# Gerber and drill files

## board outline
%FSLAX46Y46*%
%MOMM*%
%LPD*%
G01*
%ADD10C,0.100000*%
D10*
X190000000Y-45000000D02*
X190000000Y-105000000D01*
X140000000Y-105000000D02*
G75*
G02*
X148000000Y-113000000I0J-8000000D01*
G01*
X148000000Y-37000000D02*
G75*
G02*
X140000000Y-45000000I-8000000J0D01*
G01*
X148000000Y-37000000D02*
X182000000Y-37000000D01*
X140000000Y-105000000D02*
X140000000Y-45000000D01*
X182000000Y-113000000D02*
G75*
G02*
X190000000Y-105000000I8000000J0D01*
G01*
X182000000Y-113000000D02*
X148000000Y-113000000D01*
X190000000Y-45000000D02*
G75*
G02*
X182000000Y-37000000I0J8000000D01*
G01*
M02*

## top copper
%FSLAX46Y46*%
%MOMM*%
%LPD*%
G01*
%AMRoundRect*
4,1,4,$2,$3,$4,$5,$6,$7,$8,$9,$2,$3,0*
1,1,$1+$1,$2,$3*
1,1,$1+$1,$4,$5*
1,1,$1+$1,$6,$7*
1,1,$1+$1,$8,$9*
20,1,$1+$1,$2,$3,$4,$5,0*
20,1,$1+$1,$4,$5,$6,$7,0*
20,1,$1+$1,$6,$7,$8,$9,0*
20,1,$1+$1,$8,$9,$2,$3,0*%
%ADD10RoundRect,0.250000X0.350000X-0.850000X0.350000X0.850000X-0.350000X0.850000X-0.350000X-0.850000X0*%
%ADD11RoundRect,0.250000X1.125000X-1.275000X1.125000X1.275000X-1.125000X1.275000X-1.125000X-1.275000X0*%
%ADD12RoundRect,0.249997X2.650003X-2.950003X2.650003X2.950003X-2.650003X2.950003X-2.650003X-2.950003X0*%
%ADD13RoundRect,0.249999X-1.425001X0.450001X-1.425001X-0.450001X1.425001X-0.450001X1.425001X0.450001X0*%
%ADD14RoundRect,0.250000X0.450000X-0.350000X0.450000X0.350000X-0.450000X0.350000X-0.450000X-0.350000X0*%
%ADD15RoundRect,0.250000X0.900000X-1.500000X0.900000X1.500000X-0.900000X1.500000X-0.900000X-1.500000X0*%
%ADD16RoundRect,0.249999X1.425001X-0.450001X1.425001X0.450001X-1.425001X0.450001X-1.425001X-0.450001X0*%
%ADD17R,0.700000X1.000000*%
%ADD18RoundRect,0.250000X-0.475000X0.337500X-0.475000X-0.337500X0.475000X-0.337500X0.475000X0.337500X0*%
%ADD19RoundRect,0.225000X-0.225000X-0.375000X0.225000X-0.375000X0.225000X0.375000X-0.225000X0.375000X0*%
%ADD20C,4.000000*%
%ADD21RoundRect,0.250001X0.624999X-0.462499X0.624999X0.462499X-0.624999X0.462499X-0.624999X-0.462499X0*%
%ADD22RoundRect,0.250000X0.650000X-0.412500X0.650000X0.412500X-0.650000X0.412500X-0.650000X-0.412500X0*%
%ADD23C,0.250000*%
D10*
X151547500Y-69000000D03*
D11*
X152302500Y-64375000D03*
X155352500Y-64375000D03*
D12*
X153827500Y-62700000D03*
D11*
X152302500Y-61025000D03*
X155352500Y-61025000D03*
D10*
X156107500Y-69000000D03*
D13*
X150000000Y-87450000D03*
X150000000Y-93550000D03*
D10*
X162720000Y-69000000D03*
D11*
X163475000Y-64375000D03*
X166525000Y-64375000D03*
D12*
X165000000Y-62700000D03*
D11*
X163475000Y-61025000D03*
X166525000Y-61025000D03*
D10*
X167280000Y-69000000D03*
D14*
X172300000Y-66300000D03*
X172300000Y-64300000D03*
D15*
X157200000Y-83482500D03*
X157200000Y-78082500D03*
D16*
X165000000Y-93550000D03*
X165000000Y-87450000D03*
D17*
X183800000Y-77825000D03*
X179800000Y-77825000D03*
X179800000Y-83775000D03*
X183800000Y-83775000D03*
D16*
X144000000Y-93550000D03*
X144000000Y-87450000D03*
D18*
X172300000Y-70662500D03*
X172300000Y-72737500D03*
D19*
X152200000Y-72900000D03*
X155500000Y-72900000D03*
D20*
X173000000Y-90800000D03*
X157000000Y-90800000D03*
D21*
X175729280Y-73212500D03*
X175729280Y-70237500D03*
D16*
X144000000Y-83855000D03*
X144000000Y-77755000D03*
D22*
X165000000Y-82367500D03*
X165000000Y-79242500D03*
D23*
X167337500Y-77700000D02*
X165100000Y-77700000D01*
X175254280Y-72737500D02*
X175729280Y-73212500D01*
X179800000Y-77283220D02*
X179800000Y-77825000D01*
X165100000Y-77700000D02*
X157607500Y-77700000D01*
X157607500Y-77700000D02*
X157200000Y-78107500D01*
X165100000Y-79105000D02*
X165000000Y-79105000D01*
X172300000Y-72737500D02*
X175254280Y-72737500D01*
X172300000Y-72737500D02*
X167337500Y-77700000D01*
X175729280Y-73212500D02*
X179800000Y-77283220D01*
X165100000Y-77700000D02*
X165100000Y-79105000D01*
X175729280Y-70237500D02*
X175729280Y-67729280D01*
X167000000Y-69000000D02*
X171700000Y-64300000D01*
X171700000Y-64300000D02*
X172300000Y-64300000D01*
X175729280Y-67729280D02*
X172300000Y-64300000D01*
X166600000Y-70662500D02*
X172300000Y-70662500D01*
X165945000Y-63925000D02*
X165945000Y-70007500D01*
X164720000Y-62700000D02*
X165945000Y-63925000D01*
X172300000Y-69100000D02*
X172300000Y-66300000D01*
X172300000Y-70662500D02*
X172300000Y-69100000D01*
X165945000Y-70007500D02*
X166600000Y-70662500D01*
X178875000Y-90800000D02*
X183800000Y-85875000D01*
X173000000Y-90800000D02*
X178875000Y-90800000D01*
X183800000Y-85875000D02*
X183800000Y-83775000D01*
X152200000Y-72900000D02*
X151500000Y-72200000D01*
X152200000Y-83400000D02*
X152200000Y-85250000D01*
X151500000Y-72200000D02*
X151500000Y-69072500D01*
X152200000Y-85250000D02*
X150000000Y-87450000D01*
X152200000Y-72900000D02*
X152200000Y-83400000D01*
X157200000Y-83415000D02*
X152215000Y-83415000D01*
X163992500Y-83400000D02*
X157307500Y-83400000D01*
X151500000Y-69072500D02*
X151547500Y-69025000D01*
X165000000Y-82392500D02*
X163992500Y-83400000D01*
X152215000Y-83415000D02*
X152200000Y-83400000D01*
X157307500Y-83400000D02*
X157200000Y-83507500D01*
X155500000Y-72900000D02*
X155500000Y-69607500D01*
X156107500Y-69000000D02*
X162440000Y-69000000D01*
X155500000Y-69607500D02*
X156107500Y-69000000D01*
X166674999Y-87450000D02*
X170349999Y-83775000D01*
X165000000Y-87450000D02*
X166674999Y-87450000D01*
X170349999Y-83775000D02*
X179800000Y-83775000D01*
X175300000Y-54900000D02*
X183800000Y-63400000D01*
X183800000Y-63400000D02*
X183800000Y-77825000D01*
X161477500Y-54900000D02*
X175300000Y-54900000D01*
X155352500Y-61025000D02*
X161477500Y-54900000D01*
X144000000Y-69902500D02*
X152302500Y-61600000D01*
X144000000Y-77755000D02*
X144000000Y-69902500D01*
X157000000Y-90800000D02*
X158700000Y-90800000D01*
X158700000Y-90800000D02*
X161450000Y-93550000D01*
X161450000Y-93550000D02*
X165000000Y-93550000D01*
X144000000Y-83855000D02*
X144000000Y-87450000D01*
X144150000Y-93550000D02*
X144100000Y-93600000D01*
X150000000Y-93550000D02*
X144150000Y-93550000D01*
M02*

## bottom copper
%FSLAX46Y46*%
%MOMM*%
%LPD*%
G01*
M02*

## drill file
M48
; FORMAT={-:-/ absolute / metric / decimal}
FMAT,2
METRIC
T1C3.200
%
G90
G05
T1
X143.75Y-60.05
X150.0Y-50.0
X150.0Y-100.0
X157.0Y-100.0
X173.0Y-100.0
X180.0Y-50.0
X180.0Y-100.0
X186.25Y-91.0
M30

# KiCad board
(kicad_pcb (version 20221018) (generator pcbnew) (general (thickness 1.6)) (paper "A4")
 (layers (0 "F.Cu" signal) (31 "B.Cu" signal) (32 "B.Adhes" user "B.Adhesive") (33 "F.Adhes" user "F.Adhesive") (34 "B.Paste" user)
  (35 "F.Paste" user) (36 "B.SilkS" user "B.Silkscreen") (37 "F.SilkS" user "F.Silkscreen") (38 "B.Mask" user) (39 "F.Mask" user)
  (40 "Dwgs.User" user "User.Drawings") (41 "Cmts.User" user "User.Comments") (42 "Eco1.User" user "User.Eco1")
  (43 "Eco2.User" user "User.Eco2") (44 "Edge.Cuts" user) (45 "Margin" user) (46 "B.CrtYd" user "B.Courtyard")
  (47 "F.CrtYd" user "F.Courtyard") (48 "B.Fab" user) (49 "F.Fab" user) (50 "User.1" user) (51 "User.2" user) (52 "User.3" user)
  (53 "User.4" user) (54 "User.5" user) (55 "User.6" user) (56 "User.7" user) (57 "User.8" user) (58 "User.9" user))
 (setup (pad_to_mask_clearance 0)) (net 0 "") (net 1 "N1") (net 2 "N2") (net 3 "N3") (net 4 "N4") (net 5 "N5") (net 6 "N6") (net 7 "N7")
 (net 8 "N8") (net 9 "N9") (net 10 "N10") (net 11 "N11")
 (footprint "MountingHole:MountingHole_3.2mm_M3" (layer "F.Cu") (at 186.25 91)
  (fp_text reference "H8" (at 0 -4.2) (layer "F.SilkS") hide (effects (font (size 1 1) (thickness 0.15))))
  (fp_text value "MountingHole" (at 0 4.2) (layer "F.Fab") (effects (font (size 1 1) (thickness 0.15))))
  (pad "" np_thru_hole circle (at 0 0) (size 3.2 3.2) (drill 3.2) (layers "*.Cu" "*.Mask")))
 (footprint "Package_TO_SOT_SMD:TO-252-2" (layer "F.Cu") (at 153.8275 63.96 90)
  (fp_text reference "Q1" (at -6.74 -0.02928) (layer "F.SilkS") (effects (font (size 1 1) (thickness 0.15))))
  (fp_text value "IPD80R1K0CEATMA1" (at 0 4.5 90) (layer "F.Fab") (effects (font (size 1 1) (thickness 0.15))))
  (pad "1" smd roundrect (at -5.04 -2.28 90) (size 2.2 1.2) (layers "F.Cu" "F.Paste" "F.Mask") (roundrect_rratio 0.2083333333) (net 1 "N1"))
  (pad "2" smd roundrect (at -0.415 -1.525 90) (size 3.05 2.75) (layers "F.Cu" "F.Paste") (roundrect_rratio 0.09090909091) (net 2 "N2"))
  (pad "2" smd roundrect (at -0.415 1.525 90) (size 3.05 2.75) (layers "F.Cu" "F.Paste") (roundrect_rratio 0.09090909091) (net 2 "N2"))
  (pad "2" smd roundrect (at 1.26 0 90) (size 6.4 5.8) (layers "F.Cu" "F.Mask") (roundrect_rratio 0.04310293103) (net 2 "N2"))
  (pad "2" smd roundrect (at 2.935 -1.525 90) (size 3.05 2.75) (layers "F.Cu" "F.Paste") (roundrect_rratio 0.09090909091) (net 2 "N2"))
  (pad "2" smd roundrect (at 2.935 1.525 90) (size 3.05 2.75) (layers "F.Cu" "F.Paste") (roundrect_rratio 0.09090909091) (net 2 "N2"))
  (pad "3" smd roundrect (at -5.04 2.28 90) (size 2.2 1.2) (layers "F.Cu" "F.Paste" "F.Mask") (roundrect_rratio 0.2083333333) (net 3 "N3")))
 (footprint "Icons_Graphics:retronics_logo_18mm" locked (layer "F.Cu") (at 165 105)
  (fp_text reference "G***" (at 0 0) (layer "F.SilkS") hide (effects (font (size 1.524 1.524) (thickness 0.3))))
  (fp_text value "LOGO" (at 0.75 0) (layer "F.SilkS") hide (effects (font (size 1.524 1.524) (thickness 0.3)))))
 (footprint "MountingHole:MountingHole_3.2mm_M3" (layer "F.Cu") (at 150 100)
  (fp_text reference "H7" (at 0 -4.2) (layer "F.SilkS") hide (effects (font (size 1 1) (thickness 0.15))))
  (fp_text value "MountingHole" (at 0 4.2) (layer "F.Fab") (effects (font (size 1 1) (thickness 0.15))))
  (pad "" np_thru_hole circle (at 0 0) (size 3.2 3.2) (drill 3.2) (layers "*.Cu" "*.Mask")))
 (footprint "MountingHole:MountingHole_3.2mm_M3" (layer "F.Cu") (at 180 50)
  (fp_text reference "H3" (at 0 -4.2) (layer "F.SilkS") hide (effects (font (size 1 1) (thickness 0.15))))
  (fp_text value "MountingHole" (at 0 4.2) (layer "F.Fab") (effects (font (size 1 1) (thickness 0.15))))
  (pad "" np_thru_hole circle (at 0 0) (size 3.2 3.2) (drill 3.2) (layers "*.Cu" "*.Mask")))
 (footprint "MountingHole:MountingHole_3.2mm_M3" (layer "F.Cu") (at 157 100)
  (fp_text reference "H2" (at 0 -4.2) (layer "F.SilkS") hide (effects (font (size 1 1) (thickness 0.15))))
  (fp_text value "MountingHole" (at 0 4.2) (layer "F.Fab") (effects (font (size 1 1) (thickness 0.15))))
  (pad "" np_thru_hole circle (at 0 0) (size 3.2 3.2) (drill 3.2) (layers "*.Cu" "*.Mask")))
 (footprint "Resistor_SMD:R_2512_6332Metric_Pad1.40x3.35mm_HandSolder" (layer "F.Cu") (at 150 90.5 -90)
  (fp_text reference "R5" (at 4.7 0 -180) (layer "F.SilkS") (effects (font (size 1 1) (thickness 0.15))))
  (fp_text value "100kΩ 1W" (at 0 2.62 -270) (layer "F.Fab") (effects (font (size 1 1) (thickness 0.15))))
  (pad "1" smd roundrect (at -3.05 0 270) (size 1.4 3.35) (layers "F.Cu" "F.Paste" "F.Mask") (roundrect_rratio 0.1785707143) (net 1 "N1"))
  (pad "2" smd roundrect (at 3.05 0 270) (size 1.4 3.35) (layers "F.Cu" "F.Paste" "F.Mask") (roundrect_rratio 0.1785707143) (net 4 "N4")))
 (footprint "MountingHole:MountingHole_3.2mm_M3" (layer "F.Cu") (at 180 100)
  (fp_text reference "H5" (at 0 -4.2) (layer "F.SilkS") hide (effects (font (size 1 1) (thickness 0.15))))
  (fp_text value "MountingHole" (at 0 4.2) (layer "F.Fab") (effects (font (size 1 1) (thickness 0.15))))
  (pad "" np_thru_hole circle (at 0 0) (size 3.2 3.2) (drill 3.2) (layers "*.Cu" "*.Mask")))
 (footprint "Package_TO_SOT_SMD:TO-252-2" (layer "F.Cu") (at 165 63.96 90)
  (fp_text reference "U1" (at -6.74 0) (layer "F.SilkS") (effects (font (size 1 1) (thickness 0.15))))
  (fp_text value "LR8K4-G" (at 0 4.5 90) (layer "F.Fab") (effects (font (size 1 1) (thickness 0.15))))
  (pad "1" smd roundrect (at -5.04 -2.28 90) (size 2.2 1.2) (layers "F.Cu" "F.Paste" "F.Mask") (roundrect_rratio 0.2083333333) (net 3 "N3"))
  (pad "2" smd roundrect (at -0.415 -1.525 90) (size 3.05 2.75) (layers "F.Cu" "F.Paste") (roundrect_rratio 0.09090909091) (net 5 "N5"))
  (pad "2" smd roundrect (at -0.415 1.525 90) (size 3.05 2.75) (layers "F.Cu" "F.Paste") (roundrect_rratio 0.09090909091) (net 5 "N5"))
  (pad "2" smd roundrect (at 1.26 0 90) (size 6.4 5.8) (layers "F.Cu" "F.Mask") (roundrect_rratio 0.04310293103) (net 5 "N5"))
  (pad "2" smd roundrect (at 2.935 -1.525 90) (size 3.05 2.75) (layers "F.Cu" "F.Paste") (roundrect_rratio 0.09090909091) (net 5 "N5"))
  (pad "2" smd roundrect (at 2.935 1.525 90) (size 3.05 2.75) (layers "F.Cu" "F.Paste") (roundrect_rratio 0.09090909091) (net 5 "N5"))
  (pad "3" smd roundrect (at -5.04 2.28 90) (size 2.2 1.2) (layers "F.Cu" "F.Paste" "F.Mask") (roundrect_rratio 0.2083333333) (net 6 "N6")))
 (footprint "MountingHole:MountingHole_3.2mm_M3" (layer "F.Cu") (at 143.75 60.05)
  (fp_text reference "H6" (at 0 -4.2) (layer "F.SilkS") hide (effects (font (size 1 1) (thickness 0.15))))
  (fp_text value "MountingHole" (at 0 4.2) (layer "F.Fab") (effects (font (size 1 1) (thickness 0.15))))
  (pad "" np_thru_hole circle (at 0 0) (size 3.2 3.2) (drill 3.2) (layers "*.Cu" "*.Mask")))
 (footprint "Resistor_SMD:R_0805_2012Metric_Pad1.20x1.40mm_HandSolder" (layer "F.Cu") (at 172.3 65.3 90)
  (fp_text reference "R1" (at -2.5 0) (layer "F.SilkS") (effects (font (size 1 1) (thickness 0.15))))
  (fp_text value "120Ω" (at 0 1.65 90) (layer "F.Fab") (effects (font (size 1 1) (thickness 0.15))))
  (pad "1" smd roundrect (at -1 0 90) (size 1.2 1.4) (layers "F.Cu" "F.Paste" "F.Mask") (roundrect_rratio 0.2083333333) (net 5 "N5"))
  (pad "2" smd roundrect (at 1 0 90) (size 1.2 1.4) (layers "F.Cu" "F.Paste" "F.Mask") (roundrect_rratio 0.2083333333) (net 6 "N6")))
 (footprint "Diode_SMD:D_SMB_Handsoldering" (layer "F.Cu") (at 157.2 80.7825 90)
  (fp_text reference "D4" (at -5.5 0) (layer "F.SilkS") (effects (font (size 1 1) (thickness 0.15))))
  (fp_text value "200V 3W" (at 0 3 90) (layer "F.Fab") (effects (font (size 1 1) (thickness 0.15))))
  (pad "1" smd roundrect (at -2.7 0 90) (size 3.5 2.3) (layers "F.Cu" "F.Paste" "F.Mask") (roundrect_rratio 0.1086956522) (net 1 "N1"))
  (pad "2" smd roundrect (at 2.7 0 90) (size 3.5 2.3) (layers "F.Cu" "F.Paste" "F.Mask") (roundrect_rratio 0.1086956522) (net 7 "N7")))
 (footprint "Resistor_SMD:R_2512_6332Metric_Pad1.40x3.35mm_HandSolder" (layer "F.Cu") (at 165 90.5 90)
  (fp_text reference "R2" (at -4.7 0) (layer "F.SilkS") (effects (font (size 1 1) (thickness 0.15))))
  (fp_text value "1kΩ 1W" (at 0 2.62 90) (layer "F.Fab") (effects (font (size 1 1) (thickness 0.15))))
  (pad "1" smd roundrect (at -3.05 0 90) (size 1.4 3.35) (layers "F.Cu" "F.Paste" "F.Mask") (roundrect_rratio 0.1785707143) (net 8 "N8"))
  (pad "2" smd roundrect (at 3.05 0 90) (size 1.4 3.35) (layers "F.Cu" "F.Paste" "F.Mask") (roundrect_rratio 0.1785707143) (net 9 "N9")))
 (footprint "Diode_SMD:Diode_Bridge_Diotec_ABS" (layer "F.Cu") (at 181.8 80.8 -90)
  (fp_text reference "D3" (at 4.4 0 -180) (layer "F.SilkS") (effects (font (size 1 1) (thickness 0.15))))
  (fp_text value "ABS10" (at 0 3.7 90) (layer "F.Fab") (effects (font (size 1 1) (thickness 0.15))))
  (pad "1" smd rect (at -2.975 -2 270) (size 1 0.7) (layers "F.Cu" "F.Paste" "F.Mask") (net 2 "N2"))
  (pad "2" smd rect (at -2.975 2 270) (size 1 0.7) (layers "F.Cu" "F.Paste" "F.Mask") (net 7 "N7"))
  (pad "3" smd rect (at 2.975 2 270) (size 1 0.7) (layers "F.Cu" "F.Paste" "F.Mask") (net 9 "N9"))
  (pad "4" smd rect (at 2.975 -2 270) (size 1 0.7) (layers "F.Cu" "F.Paste" "F.Mask") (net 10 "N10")))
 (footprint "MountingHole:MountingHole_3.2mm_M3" (layer "F.Cu") (at 173 100)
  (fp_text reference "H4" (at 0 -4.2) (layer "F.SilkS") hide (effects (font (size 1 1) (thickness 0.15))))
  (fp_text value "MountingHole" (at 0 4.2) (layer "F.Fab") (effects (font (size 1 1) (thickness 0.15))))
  (pad "" np_thru_hole circle (at 0 0) (size 3.2 3.2) (drill 3.2) (layers "*.Cu" "*.Mask")))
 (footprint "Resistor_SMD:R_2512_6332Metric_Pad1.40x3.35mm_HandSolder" (layer "F.Cu") (at 144 90.5 90)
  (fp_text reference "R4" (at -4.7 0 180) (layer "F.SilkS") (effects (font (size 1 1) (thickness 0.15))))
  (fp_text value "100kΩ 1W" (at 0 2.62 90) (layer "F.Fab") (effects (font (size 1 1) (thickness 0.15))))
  (pad "1" smd roundrect (at -3.05 0 90) (size 1.4 3.35) (layers "F.Cu" "F.Paste" "F.Mask") (roundrect_rratio 0.1785707143) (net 4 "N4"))
  (pad "2" smd roundrect (at 3.05 0 90) (size 1.4 3.35) (layers "F.Cu" "F.Paste" "F.Mask") (roundrect_rratio 0.1785707143) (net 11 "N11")))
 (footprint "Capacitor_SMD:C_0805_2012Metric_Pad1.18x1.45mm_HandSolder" (layer "F.Cu") (at 172.3 71.7 -90)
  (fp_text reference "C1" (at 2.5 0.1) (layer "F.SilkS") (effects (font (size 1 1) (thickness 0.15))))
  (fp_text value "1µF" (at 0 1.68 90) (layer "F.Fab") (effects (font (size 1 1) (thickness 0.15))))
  (pad "1" smd roundrect (at -1.0375 0 270) (size 1.175 1.45) (layers "F.Cu" "F.Paste" "F.Mask") (roundrect_rratio 0.2127659574)
   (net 5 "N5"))
  (pad "2" smd roundrect (at 1.0375 0 270) (size 1.175 1.45) (layers "F.Cu" "F.Paste" "F.Mask") (roundrect_rratio 0.2127659574) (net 7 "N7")))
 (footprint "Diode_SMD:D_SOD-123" (layer "F.Cu") (at 153.85 72.9)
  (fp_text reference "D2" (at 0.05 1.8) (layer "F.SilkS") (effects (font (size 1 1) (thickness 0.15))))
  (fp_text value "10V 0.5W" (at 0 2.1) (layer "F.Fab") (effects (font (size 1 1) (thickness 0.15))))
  (pad "1" smd roundrect (at -1.65 0) (size 0.9 1.2) (layers "F.Cu" "F.Paste" "F.Mask") (roundrect_rratio 0.25) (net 1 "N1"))
  (pad "2" smd roundrect (at 1.65 0) (size 0.9 1.2) (layers "F.Cu" "F.Paste" "F.Mask") (roundrect_rratio 0.25) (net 3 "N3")))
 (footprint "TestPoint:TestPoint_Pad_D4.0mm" (layer "F.Cu") (at 173 90.8)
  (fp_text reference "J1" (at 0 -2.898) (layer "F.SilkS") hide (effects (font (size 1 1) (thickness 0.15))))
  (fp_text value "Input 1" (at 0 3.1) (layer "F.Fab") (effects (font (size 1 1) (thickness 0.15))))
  (pad "1" smd circle (at 0 0) (size 4 4) (layers "F.Cu" "F.Mask") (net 10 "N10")))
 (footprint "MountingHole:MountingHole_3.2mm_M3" (layer "F.Cu") (at 150 50)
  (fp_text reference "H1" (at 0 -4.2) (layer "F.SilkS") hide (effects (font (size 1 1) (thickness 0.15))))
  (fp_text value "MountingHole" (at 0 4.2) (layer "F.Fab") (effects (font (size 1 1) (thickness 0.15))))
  (pad "" np_thru_hole circle (at 0 0) (size 3.2 3.2) (drill 3.2) (layers "*.Cu" "*.Mask")))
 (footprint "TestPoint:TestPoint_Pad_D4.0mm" (layer "F.Cu") (at 157 90.8)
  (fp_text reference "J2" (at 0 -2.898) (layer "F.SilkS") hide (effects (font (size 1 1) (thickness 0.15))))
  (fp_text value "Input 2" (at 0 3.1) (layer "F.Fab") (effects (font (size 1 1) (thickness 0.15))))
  (pad "1" smd circle (at 0 0) (size 4 4) (layers "F.Cu" "F.Mask") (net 8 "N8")))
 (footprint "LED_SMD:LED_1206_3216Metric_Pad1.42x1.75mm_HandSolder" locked (layer "F.Cu") (at 175.72928 71.725 90)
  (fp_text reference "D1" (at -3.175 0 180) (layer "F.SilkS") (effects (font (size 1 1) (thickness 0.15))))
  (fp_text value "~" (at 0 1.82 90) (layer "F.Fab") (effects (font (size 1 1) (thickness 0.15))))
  (pad "1" smd roundrect locked (at -1.4875 0 90) (size 1.425 1.75) (layers "F.Cu" "F.Paste" "F.Mask") (roundrect_rratio 0.1754392982)
   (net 7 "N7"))
  (pad "2" smd roundrect locked (at 1.4875 0 90) (size 1.425 1.75) (layers "F.Cu" "F.Paste" "F.Mask") (roundrect_rratio 0.1754392982)
   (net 6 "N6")))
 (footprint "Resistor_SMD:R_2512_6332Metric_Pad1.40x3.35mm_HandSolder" (layer "F.Cu") (at 144 80.805 90)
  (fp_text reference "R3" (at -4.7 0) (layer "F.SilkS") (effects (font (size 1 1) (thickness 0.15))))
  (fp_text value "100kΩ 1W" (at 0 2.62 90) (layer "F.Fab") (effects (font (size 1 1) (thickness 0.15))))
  (pad "1" smd roundrect (at -3.05 0 90) (size 1.4 3.35) (layers "F.Cu" "F.Paste" "F.Mask") (roundrect_rratio 0.1785707143) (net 11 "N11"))
  (pad "2" smd roundrect (at 3.05 0 90) (size 1.4 3.35) (layers "F.Cu" "F.Paste" "F.Mask") (roundrect_rratio 0.1785707143) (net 2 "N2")))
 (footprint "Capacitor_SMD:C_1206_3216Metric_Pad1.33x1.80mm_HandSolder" (layer "F.Cu") (at 165 80.805 90)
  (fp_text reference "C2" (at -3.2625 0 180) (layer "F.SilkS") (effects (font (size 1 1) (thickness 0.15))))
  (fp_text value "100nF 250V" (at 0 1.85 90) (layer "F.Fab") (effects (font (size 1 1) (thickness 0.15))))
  (pad "1" smd roundrect (at -1.5625 0 90) (size 1.325 1.8) (layers "F.Cu" "F.Paste" "F.Mask") (roundrect_rratio 0.1886792453) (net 1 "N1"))
  (pad "2" smd roundrect (at 1.5625 0 90) (size 1.325 1.8) (layers "F.Cu" "F.Paste" "F.Mask") (roundrect_rratio 0.1886792453) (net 7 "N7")))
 (gr_line (start 190 45) (end 190 105) (stroke (width 0.1) (type default)) (layer "Edge.Cuts"))
 (gr_arc (start 140 105) (mid 145.656854 107.343146) (end 148 113) (stroke (width 0.1) (type default)) (layer "Edge.Cuts"))
 (gr_arc (start 148 37) (mid 145.656854 42.656854) (end 140 45) (stroke (width 0.1) (type default)) (layer "Edge.Cuts"))
 (gr_line (start 148 37) (end 182 37) (stroke (width 0.1) (type default)) (layer "Edge.Cuts"))
 (gr_line (start 140 105) (end 140 45) (stroke (width 0.1) (type default)) (layer "Edge.Cuts"))
 (gr_arc (start 182 113) (mid 184.343146 107.343146) (end 190 105) (stroke (width 0.1) (type default)) (layer "Edge.Cuts"))
 (gr_line (start 182 113) (end 148 113) (stroke (width 0.1) (type default)) (layer "Edge.Cuts"))
 (gr_arc (start 190 45) (mid 184.343146 42.656854) (end 182 37) (stroke (width 0.1) (type default)) (layer "Edge.Cuts"))
 (segment (start 167.3375 77.7) (end 165.1 77.7) (width 0.25) (layer "F.Cu") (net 7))
 (segment (start 175.25428 72.7375) (end 175.72928 73.2125) (width 0.25) (layer "F.Cu") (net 7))
 (segment (start 179.8 77.28322) (end 179.8 77.825) (width 0.25) (layer "F.Cu") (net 7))
 (segment (start 165.1 77.7) (end 157.6075 77.7) (width 0.25) (layer "F.Cu") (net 7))
 (segment (start 157.6075 77.7) (end 157.2 78.1075) (width 0.25) (layer "F.Cu") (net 7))
 (segment (start 165.1 79.105) (end 165 79.105) (width 0.25) (layer "F.Cu") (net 7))
 (segment (start 172.3 72.7375) (end 175.25428 72.7375) (width 0.25) (layer "F.Cu") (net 7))
 (segment (start 172.3 72.7375) (end 167.3375 77.7) (width 0.25) (layer "F.Cu") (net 7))
 (segment (start 175.72928 73.2125) (end 179.8 77.28322) (width 0.25) (layer "F.Cu") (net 7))
 (segment (start 165.1 77.7) (end 165.1 79.105) (width 0.25) (layer "F.Cu") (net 7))
 (segment (start 175.72928 70.2375) (end 175.72928 67.72928) (width 0.25) (layer "F.Cu") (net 6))
 (segment (start 167 69) (end 171.7 64.3) (width 0.25) (layer "F.Cu") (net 6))
 (segment (start 171.7 64.3) (end 172.3 64.3) (width 0.25) (layer "F.Cu") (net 6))
 (segment (start 175.72928 67.72928) (end 172.3 64.3) (width 0.25) (layer "F.Cu") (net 6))
 (segment (start 166.6 70.6625) (end 172.3 70.6625) (width 0.25) (layer "F.Cu") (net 5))
 (segment (start 165.945 63.925) (end 165.945 70.0075) (width 0.25) (layer "F.Cu") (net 5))
 (segment (start 164.72 62.7) (end 165.945 63.925) (width 0.25) (layer "F.Cu") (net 5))
 (segment (start 172.3 69.1) (end 172.3 66.3) (width 0.25) (layer "F.Cu") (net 5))
 (segment (start 172.3 70.6625) (end 172.3 69.1) (width 0.25) (layer "F.Cu") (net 5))
 (segment (start 165.945 70.0075) (end 166.6 70.6625) (width 0.25) (layer "F.Cu") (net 5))
 (segment (start 178.875 90.8) (end 183.8 85.875) (width 0.25) (layer "F.Cu") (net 10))
 (segment (start 173 90.8) (end 178.875 90.8) (width 0.25) (layer "F.Cu") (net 10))
 (segment (start 183.8 85.875) (end 183.8 83.775) (width 0.25) (layer "F.Cu") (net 10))
 (segment (start 152.2 72.9) (end 151.5 72.2) (width 0.25) (layer "F.Cu") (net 1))
 (segment (start 152.2 83.4) (end 152.2 85.25) (width 0.25) (layer "F.Cu") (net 1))
 (segment (start 151.5 72.2) (end 151.5 69.0725) (width 0.25) (layer "F.Cu") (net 1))
 (segment (start 152.2 85.25) (end 150 87.45) (width 0.25) (layer "F.Cu") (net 1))
 (segment (start 152.2 72.9) (end 152.2 83.4) (width 0.25) (layer "F.Cu") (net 1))
 (segment (start 157.2 83.415) (end 152.215 83.415) (width 0.25) (layer "F.Cu") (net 1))
 (segment (start 163.9925 83.4) (end 157.3075 83.4) (width 0.25) (layer "F.Cu") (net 1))
 (segment (start 151.5 69.0725) (end 151.5475 69.025) (width 0.25) (layer "F.Cu") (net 1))
 (segment (start 165 82.3925) (end 163.9925 83.4) (width 0.25) (layer "F.Cu") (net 1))
 (segment (start 152.215 83.415) (end 152.2 83.4) (width 0.25) (layer "F.Cu") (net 1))
 (segment (start 157.3075 83.4) (end 157.2 83.5075) (width 0.25) (layer "F.Cu") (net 1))
 (segment (start 155.5 72.9) (end 155.5 69.6075) (width 0.25) (layer "F.Cu") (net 3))
 (segment (start 156.1075 69) (end 162.44 69) (width 0.25) (layer "F.Cu") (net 3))
 (segment (start 155.5 69.6075) (end 156.1075 69) (width 0.25) (layer "F.Cu") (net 3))
 (segment (start 166.674999 87.45) (end 170.349999 83.775) (width 0.25) (layer "F.Cu") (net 9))
 (segment (start 165 87.45) (end 166.674999 87.45) (width 0.25) (layer "F.Cu") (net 9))
 (segment (start 170.349999 83.775) (end 179.8 83.775) (width 0.25) (layer "F.Cu") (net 9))
 (segment (start 175.3 54.9) (end 183.8 63.4) (width 0.25) (layer "F.Cu") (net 2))
 (segment (start 183.8 63.4) (end 183.8 77.825) (width 0.25) (layer "F.Cu") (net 2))
 (segment (start 161.4775 54.9) (end 175.3 54.9) (width 0.25) (layer "F.Cu") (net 2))
 (segment (start 155.3525 61.025) (end 161.4775 54.9) (width 0.25) (layer "F.Cu") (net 2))
 (segment (start 144 69.9025) (end 152.3025 61.6) (width 0.25) (layer "F.Cu") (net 2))
 (segment (start 144 77.755) (end 144 69.9025) (width 0.25) (layer "F.Cu") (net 2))
 (segment (start 157 90.8) (end 158.7 90.8) (width 0.25) (layer "F.Cu") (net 8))
 (segment (start 158.7 90.8) (end 161.45 93.55) (width 0.25) (layer "F.Cu") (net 8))
 (segment (start 161.45 93.55) (end 165 93.55) (width 0.25) (layer "F.Cu") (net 8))
 (segment (start 144 83.855) (end 144 87.45) (width 0.25) (layer "F.Cu") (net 11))
 (segment (start 144.15 93.55) (end 144.1 93.6) (width 0.25) (layer "F.Cu") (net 4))
 (segment (start 150 93.55) (end 144.15 93.55) (width 0.25) (layer "F.Cu") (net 4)))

